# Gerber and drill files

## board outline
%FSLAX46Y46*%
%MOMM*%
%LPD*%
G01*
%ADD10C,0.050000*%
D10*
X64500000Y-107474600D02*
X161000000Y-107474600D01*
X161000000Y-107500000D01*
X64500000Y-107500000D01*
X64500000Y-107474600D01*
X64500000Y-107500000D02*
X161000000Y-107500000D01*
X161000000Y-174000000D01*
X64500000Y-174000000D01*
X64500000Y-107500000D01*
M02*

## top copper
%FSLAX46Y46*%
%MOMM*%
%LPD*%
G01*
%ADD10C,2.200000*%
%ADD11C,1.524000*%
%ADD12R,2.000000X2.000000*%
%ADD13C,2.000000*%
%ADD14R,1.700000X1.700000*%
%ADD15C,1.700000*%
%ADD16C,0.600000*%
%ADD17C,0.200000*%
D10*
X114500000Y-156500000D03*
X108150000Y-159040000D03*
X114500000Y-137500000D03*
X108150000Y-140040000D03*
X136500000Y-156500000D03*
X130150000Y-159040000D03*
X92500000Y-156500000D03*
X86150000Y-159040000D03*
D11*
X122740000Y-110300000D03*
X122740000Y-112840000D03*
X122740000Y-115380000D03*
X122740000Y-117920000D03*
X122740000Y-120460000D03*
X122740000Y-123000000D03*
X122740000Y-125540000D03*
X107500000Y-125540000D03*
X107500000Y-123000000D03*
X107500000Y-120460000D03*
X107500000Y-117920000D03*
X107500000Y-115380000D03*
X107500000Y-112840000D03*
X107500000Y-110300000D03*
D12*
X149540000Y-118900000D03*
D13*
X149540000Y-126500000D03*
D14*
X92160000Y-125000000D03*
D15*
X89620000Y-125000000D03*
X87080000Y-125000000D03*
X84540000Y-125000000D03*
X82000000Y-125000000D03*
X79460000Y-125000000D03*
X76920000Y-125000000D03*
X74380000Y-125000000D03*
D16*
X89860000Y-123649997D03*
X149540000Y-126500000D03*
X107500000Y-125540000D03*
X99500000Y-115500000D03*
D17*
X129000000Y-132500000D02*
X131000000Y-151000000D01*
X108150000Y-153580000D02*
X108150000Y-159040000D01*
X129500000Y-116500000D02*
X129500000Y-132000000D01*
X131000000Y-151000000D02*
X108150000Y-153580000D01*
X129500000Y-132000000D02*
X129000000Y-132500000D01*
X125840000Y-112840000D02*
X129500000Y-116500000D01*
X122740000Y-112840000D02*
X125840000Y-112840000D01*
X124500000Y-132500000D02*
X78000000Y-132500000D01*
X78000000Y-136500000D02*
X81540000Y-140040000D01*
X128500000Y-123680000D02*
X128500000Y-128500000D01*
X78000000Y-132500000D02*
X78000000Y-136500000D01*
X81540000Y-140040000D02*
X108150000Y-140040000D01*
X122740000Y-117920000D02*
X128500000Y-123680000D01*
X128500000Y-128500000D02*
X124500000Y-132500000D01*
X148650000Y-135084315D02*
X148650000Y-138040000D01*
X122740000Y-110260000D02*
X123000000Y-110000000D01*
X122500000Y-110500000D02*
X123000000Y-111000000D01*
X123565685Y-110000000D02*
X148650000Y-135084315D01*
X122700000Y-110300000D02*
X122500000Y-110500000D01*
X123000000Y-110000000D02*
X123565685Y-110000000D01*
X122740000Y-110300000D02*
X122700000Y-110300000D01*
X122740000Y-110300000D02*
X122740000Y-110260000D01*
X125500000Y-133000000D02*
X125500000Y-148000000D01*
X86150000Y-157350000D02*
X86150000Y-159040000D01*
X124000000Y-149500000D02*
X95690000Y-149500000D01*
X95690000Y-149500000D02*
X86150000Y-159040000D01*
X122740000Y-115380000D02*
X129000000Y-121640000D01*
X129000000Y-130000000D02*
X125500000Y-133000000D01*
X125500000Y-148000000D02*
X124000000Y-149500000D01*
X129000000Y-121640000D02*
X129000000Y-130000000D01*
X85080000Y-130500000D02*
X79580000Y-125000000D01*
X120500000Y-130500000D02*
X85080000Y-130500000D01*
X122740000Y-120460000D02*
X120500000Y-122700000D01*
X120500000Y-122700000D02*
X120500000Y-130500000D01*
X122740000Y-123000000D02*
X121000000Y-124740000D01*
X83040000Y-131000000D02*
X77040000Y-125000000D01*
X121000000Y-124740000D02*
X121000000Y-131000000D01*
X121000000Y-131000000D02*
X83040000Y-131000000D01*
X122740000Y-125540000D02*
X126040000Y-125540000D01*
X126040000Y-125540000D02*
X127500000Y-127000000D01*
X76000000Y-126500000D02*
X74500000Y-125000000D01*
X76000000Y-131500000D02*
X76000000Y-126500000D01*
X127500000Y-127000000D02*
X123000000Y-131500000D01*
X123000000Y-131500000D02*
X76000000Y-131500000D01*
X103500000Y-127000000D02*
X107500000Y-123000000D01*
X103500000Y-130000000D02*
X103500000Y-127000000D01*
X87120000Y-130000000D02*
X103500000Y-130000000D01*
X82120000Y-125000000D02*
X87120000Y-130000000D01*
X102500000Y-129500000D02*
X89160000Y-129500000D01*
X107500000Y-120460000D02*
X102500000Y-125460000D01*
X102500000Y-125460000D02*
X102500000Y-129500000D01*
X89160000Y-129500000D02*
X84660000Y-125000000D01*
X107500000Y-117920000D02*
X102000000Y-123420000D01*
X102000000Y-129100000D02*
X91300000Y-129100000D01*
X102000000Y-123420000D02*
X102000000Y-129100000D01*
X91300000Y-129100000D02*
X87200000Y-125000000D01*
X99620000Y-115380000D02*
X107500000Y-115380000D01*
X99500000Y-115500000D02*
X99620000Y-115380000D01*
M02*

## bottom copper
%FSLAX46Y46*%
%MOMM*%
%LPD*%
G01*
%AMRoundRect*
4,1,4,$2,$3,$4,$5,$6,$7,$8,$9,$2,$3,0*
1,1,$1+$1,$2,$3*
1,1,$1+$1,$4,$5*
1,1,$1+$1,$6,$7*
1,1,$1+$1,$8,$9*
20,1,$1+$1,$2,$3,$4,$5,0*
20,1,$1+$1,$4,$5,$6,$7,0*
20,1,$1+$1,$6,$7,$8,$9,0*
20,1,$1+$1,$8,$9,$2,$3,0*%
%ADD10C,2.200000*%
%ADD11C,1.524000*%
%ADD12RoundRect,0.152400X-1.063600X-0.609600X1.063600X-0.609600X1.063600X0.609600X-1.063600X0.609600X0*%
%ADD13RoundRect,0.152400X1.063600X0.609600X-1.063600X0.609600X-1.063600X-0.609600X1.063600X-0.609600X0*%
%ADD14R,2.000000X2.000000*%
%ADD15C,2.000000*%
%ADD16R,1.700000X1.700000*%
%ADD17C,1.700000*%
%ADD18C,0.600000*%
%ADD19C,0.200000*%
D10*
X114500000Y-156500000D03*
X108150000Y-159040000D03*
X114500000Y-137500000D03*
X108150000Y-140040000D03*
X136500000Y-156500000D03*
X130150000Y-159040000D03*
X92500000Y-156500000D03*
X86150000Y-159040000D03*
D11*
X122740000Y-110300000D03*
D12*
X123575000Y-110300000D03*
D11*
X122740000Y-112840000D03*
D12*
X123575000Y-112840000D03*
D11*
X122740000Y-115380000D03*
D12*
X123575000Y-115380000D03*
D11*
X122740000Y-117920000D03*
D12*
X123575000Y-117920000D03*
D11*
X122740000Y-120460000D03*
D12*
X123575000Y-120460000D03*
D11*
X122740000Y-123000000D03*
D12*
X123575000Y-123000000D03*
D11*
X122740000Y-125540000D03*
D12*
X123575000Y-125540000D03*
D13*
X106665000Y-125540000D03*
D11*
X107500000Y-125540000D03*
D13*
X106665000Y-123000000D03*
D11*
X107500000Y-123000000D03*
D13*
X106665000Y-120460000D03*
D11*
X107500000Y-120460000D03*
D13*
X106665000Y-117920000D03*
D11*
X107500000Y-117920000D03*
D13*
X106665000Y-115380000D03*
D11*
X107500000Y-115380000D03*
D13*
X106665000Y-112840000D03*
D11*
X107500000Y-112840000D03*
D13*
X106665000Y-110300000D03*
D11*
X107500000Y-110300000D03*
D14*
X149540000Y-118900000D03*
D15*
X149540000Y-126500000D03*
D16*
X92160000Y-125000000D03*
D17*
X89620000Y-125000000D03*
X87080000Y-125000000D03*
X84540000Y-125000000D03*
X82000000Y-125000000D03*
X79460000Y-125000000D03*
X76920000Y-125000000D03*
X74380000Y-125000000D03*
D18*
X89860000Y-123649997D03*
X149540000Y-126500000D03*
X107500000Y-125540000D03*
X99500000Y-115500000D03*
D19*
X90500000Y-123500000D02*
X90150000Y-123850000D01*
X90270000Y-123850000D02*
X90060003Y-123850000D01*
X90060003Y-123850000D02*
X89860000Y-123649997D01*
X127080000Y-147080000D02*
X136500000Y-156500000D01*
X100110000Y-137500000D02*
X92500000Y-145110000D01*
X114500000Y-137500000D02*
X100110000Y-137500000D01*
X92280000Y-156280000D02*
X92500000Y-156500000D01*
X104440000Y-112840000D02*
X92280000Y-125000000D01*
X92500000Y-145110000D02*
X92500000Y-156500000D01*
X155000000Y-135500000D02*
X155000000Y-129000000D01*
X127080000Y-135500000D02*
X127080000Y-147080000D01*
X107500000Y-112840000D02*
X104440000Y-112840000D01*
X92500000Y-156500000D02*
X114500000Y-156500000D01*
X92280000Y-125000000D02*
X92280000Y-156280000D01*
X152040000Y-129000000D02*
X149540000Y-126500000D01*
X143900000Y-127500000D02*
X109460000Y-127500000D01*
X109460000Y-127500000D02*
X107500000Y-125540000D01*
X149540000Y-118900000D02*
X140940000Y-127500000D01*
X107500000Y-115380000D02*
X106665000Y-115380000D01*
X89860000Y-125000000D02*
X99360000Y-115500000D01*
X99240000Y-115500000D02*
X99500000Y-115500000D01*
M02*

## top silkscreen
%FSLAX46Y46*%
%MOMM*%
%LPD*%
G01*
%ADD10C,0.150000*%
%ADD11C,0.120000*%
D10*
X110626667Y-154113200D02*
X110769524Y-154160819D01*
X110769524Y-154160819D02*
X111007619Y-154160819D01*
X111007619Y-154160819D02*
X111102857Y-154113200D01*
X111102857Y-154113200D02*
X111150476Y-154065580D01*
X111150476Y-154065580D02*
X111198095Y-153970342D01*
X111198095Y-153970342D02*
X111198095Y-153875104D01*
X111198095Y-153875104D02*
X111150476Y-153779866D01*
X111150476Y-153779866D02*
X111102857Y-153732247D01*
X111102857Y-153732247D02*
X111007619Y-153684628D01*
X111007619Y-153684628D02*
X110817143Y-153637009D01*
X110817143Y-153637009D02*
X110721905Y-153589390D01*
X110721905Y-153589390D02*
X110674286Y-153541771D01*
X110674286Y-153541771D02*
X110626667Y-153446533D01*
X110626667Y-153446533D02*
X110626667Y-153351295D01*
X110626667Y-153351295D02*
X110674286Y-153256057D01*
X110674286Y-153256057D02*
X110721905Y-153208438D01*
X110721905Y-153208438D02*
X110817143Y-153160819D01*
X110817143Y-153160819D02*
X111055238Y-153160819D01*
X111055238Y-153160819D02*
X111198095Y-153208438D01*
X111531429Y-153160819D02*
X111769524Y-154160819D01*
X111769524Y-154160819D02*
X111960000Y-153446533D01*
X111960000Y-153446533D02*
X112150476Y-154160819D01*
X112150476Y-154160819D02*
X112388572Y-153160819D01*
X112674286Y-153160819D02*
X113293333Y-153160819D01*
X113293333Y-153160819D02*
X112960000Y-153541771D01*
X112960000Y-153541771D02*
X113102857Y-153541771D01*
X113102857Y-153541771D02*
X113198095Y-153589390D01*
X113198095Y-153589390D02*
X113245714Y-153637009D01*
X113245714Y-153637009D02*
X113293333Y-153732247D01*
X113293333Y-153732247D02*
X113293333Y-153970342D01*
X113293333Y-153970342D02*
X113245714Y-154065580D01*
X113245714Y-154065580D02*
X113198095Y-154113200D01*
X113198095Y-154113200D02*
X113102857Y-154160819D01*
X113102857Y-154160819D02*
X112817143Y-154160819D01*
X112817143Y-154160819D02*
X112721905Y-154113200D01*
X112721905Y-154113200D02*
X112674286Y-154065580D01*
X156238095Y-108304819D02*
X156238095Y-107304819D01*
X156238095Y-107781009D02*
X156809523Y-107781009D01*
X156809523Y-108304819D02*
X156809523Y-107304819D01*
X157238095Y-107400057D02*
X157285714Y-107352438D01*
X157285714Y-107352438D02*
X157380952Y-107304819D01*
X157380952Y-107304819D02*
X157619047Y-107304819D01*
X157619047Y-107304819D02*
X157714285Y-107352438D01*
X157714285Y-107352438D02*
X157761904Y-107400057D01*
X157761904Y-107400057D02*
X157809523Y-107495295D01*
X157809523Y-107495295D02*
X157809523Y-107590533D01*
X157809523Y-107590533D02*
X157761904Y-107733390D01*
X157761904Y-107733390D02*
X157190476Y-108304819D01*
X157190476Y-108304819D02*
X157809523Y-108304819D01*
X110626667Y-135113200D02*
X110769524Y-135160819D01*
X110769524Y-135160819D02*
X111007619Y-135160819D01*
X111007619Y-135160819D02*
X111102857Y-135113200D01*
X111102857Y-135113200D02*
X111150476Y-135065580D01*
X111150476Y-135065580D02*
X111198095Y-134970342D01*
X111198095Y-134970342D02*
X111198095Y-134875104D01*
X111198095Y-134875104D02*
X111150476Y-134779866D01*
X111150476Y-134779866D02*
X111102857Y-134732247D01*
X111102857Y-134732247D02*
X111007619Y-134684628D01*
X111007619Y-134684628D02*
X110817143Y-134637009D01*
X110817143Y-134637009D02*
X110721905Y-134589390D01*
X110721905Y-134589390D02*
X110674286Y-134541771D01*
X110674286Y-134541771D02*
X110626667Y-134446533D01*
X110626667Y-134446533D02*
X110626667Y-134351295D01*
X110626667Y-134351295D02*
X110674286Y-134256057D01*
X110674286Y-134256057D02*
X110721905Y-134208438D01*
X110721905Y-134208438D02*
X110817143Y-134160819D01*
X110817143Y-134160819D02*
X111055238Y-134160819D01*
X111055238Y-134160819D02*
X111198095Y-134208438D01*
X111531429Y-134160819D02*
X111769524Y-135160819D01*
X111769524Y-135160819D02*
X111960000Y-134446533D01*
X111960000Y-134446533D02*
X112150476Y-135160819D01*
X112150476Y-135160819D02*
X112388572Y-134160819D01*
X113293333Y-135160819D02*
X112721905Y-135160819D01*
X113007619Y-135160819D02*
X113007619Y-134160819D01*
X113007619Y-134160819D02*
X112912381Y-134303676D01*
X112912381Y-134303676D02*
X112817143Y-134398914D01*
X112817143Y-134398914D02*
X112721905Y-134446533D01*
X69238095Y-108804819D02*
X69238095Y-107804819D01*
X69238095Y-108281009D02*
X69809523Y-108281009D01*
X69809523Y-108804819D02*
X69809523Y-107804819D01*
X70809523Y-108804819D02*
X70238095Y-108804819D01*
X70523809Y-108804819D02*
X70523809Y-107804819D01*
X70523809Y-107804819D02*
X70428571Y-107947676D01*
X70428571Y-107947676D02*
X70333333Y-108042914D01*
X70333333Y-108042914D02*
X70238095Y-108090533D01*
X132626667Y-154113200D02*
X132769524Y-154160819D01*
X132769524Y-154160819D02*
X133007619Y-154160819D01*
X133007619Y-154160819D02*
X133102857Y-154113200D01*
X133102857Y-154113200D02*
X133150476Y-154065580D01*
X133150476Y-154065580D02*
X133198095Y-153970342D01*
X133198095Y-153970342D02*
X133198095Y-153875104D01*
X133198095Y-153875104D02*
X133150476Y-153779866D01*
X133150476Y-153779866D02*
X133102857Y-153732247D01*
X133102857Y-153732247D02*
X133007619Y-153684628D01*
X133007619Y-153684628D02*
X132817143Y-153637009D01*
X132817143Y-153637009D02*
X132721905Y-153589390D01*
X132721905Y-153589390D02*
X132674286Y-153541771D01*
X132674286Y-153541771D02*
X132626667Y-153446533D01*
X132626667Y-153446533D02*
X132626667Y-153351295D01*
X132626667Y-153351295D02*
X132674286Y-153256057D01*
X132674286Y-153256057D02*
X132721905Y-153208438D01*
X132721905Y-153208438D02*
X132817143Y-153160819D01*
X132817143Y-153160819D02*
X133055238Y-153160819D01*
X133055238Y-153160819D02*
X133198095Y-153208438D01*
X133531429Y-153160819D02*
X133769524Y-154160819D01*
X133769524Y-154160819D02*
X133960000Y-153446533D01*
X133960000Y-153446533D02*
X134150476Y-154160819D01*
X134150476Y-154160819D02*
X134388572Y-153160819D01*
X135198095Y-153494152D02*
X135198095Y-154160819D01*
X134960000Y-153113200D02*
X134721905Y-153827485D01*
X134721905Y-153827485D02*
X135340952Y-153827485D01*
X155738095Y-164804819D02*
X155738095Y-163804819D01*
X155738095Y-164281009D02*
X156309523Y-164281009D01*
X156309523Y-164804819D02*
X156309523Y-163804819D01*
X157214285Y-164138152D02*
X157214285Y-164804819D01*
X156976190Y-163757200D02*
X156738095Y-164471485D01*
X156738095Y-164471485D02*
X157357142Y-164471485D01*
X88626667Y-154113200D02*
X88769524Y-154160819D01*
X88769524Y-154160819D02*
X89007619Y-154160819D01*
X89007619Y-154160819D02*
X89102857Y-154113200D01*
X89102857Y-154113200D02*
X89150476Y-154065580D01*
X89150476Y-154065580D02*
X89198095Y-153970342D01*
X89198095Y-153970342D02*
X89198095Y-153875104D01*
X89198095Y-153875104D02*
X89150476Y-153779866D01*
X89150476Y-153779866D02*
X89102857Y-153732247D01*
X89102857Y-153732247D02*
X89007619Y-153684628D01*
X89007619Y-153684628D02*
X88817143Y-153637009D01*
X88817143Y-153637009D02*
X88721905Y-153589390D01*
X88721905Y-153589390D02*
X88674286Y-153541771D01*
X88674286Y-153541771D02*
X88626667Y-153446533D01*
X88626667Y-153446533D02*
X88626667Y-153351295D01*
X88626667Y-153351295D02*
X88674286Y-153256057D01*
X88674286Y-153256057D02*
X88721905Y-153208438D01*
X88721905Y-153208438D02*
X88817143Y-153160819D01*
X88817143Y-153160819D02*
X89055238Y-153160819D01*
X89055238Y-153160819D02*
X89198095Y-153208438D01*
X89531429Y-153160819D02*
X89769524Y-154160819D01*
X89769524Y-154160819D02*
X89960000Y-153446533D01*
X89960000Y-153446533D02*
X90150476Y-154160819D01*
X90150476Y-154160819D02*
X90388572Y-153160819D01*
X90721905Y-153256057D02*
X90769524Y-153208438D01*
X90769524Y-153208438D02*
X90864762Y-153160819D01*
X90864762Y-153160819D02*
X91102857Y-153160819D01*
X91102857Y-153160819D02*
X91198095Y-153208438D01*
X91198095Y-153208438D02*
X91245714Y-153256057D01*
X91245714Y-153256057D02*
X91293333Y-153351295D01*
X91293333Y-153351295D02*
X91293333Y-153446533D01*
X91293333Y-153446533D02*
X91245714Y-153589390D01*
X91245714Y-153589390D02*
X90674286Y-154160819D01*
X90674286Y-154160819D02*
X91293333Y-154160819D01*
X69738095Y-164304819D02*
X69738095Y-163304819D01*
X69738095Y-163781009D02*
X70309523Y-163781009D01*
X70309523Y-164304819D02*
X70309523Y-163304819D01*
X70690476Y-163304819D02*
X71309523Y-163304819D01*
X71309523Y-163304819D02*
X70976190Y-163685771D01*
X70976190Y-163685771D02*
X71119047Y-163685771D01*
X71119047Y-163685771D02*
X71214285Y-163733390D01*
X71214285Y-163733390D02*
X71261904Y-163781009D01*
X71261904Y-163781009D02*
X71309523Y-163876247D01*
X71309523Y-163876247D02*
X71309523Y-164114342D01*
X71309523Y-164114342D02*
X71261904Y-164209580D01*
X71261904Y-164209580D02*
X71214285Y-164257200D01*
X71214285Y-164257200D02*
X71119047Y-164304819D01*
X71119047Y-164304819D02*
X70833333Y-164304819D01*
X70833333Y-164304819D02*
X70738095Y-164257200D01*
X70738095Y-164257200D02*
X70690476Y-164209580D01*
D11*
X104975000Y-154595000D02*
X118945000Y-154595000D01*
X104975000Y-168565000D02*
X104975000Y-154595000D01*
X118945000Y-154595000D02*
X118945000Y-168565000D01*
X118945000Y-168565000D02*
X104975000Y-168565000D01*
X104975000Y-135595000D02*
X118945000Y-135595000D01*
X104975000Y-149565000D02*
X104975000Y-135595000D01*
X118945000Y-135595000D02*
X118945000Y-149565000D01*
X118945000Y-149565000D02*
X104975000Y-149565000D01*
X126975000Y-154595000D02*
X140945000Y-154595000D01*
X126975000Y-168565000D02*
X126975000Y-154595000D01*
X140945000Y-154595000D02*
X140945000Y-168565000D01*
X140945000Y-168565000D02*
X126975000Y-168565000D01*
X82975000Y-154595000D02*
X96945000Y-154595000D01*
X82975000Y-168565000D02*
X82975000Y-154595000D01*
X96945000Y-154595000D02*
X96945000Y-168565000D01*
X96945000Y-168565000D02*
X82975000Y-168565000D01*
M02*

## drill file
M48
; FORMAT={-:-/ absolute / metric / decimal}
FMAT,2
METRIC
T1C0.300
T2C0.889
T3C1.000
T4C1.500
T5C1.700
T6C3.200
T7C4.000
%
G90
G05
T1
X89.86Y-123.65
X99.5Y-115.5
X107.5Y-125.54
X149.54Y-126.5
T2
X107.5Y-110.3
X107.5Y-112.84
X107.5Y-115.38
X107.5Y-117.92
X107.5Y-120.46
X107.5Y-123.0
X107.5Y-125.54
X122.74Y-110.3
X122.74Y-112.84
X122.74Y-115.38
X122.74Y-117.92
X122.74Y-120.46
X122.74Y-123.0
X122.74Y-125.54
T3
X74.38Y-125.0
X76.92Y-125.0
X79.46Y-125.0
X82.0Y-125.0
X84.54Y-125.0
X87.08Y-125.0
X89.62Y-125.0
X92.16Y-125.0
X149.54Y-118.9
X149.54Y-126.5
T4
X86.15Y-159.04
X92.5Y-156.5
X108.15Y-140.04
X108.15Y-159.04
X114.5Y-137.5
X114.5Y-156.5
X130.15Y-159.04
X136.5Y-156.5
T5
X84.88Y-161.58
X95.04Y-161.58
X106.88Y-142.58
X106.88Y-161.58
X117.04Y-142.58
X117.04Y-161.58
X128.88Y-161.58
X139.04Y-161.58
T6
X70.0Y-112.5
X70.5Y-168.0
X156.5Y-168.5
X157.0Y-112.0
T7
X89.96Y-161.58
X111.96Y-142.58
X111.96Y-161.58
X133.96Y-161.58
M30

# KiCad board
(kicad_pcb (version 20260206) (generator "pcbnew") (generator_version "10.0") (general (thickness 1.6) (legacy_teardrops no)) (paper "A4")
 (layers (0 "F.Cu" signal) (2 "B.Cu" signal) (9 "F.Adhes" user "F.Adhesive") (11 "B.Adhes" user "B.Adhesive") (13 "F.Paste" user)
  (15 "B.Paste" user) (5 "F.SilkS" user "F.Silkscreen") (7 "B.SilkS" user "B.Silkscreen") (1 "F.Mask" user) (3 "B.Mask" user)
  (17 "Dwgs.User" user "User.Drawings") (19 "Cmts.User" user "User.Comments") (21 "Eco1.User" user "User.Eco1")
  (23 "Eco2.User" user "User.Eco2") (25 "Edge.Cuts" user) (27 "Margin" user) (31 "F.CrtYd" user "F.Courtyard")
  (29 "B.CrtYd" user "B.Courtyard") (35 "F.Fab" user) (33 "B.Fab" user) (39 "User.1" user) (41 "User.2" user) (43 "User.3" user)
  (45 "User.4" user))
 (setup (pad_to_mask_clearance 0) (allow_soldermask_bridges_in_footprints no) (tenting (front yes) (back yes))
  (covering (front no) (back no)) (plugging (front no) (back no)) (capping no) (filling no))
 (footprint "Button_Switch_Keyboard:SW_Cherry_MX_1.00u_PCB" (layer "F.Cu") (at 114.5 156.5)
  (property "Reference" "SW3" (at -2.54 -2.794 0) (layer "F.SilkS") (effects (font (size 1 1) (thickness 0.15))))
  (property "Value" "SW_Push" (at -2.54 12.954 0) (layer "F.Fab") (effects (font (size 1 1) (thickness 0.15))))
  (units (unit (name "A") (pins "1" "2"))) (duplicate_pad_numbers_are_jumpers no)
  (fp_line (start -9.525 -1.905) (end 4.445 -1.905) (stroke (width 0.12) (type solid)) (layer "F.SilkS"))
  (fp_line (start -9.525 12.065) (end -9.525 -1.905) (stroke (width 0.12) (type solid)) (layer "F.SilkS"))
  (fp_line (start 4.445 -1.905) (end 4.445 12.065) (stroke (width 0.12) (type solid)) (layer "F.SilkS"))
  (fp_line (start 4.445 12.065) (end -9.525 12.065) (stroke (width 0.12) (type solid)) (layer "F.SilkS"))
  (pad "" np_thru_hole circle (at -7.62 5.08) (size 1.7 1.7) (drill 1.7) (layers "*.Cu" "*.Mask"))
  (pad "" np_thru_hole circle (at -2.54 5.08) (size 4 4) (drill 4) (layers "*.Cu" "*.Mask"))
  (pad "" np_thru_hole circle (at 2.54 5.08) (size 1.7 1.7) (drill 1.7) (layers "*.Cu" "*.Mask"))
  (pad "1" thru_hole circle (at 0 0) (size 2.2 2.2) (drill 1.5) (layers "*.Cu" "*.Mask") (remove_unused_layers no) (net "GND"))
  (pad "2" thru_hole circle (at -6.35 2.54) (size 2.2 2.2) (drill 1.5) (layers "*.Cu" "*.Mask") (remove_unused_layers no)
   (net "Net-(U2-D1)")))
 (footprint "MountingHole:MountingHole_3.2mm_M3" (layer "F.Cu") (at 157 112)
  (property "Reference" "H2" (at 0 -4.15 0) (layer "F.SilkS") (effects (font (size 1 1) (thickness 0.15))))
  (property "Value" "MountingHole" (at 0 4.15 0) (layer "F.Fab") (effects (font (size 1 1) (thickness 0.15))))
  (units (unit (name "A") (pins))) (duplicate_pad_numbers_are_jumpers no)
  (pad "" np_thru_hole circle (at 0 0) (size 3.2 3.2) (drill 3.2) (layers "*.Cu" "*.Mask")))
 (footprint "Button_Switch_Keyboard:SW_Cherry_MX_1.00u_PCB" (layer "F.Cu") (at 114.5 137.5)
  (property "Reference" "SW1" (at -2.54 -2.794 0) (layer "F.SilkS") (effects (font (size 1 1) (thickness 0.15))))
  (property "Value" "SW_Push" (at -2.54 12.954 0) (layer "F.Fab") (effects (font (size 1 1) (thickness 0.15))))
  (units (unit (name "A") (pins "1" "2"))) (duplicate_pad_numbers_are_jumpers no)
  (fp_line (start -9.525 -1.905) (end 4.445 -1.905) (stroke (width 0.12) (type solid)) (layer "F.SilkS"))
  (fp_line (start -9.525 12.065) (end -9.525 -1.905) (stroke (width 0.12) (type solid)) (layer "F.SilkS"))
  (fp_line (start 4.445 -1.905) (end 4.445 12.065) (stroke (width 0.12) (type solid)) (layer "F.SilkS"))
  (fp_line (start 4.445 12.065) (end -9.525 12.065) (stroke (width 0.12) (type solid)) (layer "F.SilkS"))
  (pad "" np_thru_hole circle (at -7.62 5.08) (size 1.7 1.7) (drill 1.7) (layers "*.Cu" "*.Mask"))
  (pad "" np_thru_hole circle (at -2.54 5.08) (size 4 4) (drill 4) (layers "*.Cu" "*.Mask"))
  (pad "" np_thru_hole circle (at 2.54 5.08) (size 1.7 1.7) (drill 1.7) (layers "*.Cu" "*.Mask"))
  (pad "1" thru_hole circle (at 0 0) (size 2.2 2.2) (drill 1.5) (layers "*.Cu" "*.Mask") (remove_unused_layers no) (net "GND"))
  (pad "2" thru_hole circle (at -6.35 2.54) (size 2.2 2.2) (drill 1.5) (layers "*.Cu" "*.Mask") (remove_unused_layers no)
   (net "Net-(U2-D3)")))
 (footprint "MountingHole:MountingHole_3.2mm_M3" (layer "F.Cu") (at 70 112.5)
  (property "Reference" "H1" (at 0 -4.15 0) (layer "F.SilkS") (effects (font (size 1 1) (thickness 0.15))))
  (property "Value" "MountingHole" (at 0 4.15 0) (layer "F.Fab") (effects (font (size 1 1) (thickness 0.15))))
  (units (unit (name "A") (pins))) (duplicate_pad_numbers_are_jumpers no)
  (pad "" np_thru_hole circle (at 0 0) (size 3.2 3.2) (drill 3.2) (layers "*.Cu" "*.Mask")))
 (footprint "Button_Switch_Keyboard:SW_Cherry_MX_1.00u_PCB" (layer "F.Cu") (at 136.5 156.5)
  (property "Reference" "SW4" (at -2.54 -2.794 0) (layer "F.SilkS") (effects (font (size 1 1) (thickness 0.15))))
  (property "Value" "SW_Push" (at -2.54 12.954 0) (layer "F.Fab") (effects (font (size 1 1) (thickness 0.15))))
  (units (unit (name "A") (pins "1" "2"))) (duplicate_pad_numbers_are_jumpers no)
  (fp_line (start -9.525 -1.905) (end 4.445 -1.905) (stroke (width 0.12) (type solid)) (layer "F.SilkS"))
  (fp_line (start -9.525 12.065) (end -9.525 -1.905) (stroke (width 0.12) (type solid)) (layer "F.SilkS"))
  (fp_line (start 4.445 -1.905) (end 4.445 12.065) (stroke (width 0.12) (type solid)) (layer "F.SilkS"))
  (fp_line (start 4.445 12.065) (end -9.525 12.065) (stroke (width 0.12) (type solid)) (layer "F.SilkS"))
  (pad "" np_thru_hole circle (at -7.62 5.08) (size 1.7 1.7) (drill 1.7) (layers "*.Cu" "*.Mask"))
  (pad "" np_thru_hole circle (at -2.54 5.08) (size 4 4) (drill 4) (layers "*.Cu" "*.Mask"))
  (pad "" np_thru_hole circle (at 2.54 5.08) (size 1.7 1.7) (drill 1.7) (layers "*.Cu" "*.Mask"))
  (pad "1" thru_hole circle (at 0 0) (size 2.2 2.2) (drill 1.5) (layers "*.Cu" "*.Mask") (remove_unused_layers no) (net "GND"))
  (pad "2" thru_hole circle (at -6.35 2.54) (size 2.2 2.2) (drill 1.5) (layers "*.Cu" "*.Mask") (remove_unused_layers no)
   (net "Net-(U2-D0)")))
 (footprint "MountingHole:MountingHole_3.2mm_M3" (layer "F.Cu") (at 156.5 168.5)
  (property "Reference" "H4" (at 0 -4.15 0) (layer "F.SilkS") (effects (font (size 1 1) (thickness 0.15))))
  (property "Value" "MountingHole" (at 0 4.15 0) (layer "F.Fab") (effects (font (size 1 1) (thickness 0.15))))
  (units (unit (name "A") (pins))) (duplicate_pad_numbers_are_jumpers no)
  (pad "" np_thru_hole circle (at 0 0) (size 3.2 3.2) (drill 3.2) (layers "*.Cu" "*.Mask")))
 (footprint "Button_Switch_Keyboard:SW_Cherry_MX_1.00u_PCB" (layer "F.Cu") (at 92.5 156.5)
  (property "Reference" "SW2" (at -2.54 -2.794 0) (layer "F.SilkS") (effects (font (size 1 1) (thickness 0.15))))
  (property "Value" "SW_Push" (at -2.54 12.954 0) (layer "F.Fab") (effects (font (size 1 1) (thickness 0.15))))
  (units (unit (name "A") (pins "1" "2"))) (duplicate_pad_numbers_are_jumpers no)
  (fp_line (start -9.525 -1.905) (end 4.445 -1.905) (stroke (width 0.12) (type solid)) (layer "F.SilkS"))
  (fp_line (start -9.525 12.065) (end -9.525 -1.905) (stroke (width 0.12) (type solid)) (layer "F.SilkS"))
  (fp_line (start 4.445 -1.905) (end 4.445 12.065) (stroke (width 0.12) (type solid)) (layer "F.SilkS"))
  (fp_line (start 4.445 12.065) (end -9.525 12.065) (stroke (width 0.12) (type solid)) (layer "F.SilkS"))
  (pad "" np_thru_hole circle (at -7.62 5.08) (size 1.7 1.7) (drill 1.7) (layers "*.Cu" "*.Mask"))
  (pad "" np_thru_hole circle (at -2.54 5.08) (size 4 4) (drill 4) (layers "*.Cu" "*.Mask"))
  (pad "" np_thru_hole circle (at 2.54 5.08) (size 1.7 1.7) (drill 1.7) (layers "*.Cu" "*.Mask"))
  (pad "1" thru_hole circle (at 0 0) (size 2.2 2.2) (drill 1.5) (layers "*.Cu" "*.Mask") (remove_unused_layers no) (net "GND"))
  (pad "2" thru_hole circle (at -6.35 2.54) (size 2.2 2.2) (drill 1.5) (layers "*.Cu" "*.Mask") (remove_unused_layers no)
   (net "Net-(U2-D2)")))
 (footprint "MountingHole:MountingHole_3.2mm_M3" (layer "F.Cu") (at 70.5 168)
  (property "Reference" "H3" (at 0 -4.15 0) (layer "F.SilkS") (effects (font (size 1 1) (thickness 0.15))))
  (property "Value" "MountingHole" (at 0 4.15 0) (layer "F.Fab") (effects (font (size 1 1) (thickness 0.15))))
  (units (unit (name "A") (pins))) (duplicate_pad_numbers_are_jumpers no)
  (pad "" np_thru_hole circle (at 0 0) (size 3.2 3.2) (drill 3.2) (layers "*.Cu" "*.Mask")))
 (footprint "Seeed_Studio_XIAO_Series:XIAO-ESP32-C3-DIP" (layer "B.Cu") (at 115.12 117.92 90)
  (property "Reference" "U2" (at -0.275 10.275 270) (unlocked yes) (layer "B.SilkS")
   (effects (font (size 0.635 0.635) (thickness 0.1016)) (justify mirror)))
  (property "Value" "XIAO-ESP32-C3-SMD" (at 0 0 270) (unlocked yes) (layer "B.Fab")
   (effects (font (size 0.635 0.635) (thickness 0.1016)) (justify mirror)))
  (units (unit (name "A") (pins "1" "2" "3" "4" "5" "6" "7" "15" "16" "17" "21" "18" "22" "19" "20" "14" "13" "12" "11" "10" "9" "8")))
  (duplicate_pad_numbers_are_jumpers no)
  (pad "1" thru_hole circle (at 7.62 7.62) (size 1.524 1.524) (drill 0.889) (layers "*.Cu" "*.Mask") (remove_unused_layers no)
   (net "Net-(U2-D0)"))
  (pad "1" smd roundrect (at 7.62 8.455) (size 2.432 1.524) (layers "B.Cu" "B.Mask") (roundrect_rratio 0.1) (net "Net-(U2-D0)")
   (thermal_bridge_angle 45))
  (pad "2" thru_hole circle (at 5.08 7.62) (size 1.524 1.524) (drill 0.889) (layers "*.Cu" "*.Mask") (remove_unused_layers no)
   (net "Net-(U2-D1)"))
  (pad "2" smd roundrect (at 5.08 8.455) (size 2.432 1.524) (layers "B.Cu" "B.Mask") (roundrect_rratio 0.1) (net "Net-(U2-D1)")
   (thermal_bridge_angle 45))
  (pad "3" thru_hole circle (at 2.54 7.62) (size 1.524 1.524) (drill 0.889) (layers "*.Cu" "*.Mask") (remove_unused_layers no)
   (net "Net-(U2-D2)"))
  (pad "3" smd roundrect (at 2.54 8.455) (size 2.432 1.524) (layers "B.Cu" "B.Mask") (roundrect_rratio 0.1) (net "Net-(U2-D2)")
   (thermal_bridge_angle 45))
  (pad "4" thru_hole circle (at 0 7.62) (size 1.524 1.524) (drill 0.889) (layers "*.Cu" "*.Mask") (remove_unused_layers no)
   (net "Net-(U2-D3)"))
  (pad "4" smd roundrect (at 0 8.455) (size 2.432 1.524) (layers "B.Cu" "B.Mask") (roundrect_rratio 0.1) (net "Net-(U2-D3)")
   (thermal_bridge_angle 45))
  (pad "5" thru_hole circle (at -2.54 7.62) (size 1.524 1.524) (drill 0.889) (layers "*.Cu" "*.Mask") (remove_unused_layers no) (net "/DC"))
  (pad "5" smd roundrect (at -2.54 8.455) (size 2.432 1.524) (layers "B.Cu" "B.Mask") (roundrect_rratio 0.1) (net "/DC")
   (thermal_bridge_angle 45))
  (pad "6" thru_hole circle (at -5.08 7.62) (size 1.524 1.524) (drill 0.889) (layers "*.Cu" "*.Mask") (remove_unused_layers no) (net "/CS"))
  (pad "6" smd roundrect (at -5.08 8.455) (size 2.432 1.524) (layers "B.Cu" "B.Mask") (roundrect_rratio 0.1) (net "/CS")
   (thermal_bridge_angle 45))
  (pad "7" thru_hole circle (at -7.62 7.62) (size 1.524 1.524) (drill 0.889) (layers "*.Cu" "*.Mask") (remove_unused_layers no) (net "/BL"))
  (pad "7" smd roundrect (at -7.62 8.455) (size 2.432 1.524) (layers "B.Cu" "B.Mask") (roundrect_rratio 0.1) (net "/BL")
   (thermal_bridge_angle 45))
  (pad "8" smd roundrect (at -7.62 -8.455 180) (size 2.432 1.524) (layers "B.Cu" "B.Mask") (roundrect_rratio 0.1) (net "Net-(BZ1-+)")
   (thermal_bridge_angle 45))
  (pad "8" thru_hole circle (at -7.62 -7.62 180) (size 1.524 1.524) (drill 0.889) (layers "*.Cu" "*.Mask") (remove_unused_layers no)
   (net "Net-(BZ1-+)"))
  (pad "9" smd roundrect (at -5.08 -8.455 180) (size 2.432 1.524) (layers "B.Cu" "B.Mask") (roundrect_rratio 0.1) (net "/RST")
   (thermal_bridge_angle 45))
  (pad "9" thru_hole circle (at -5.08 -7.62 180) (size 1.524 1.524) (drill 0.889) (layers "*.Cu" "*.Mask") (remove_unused_layers no)
   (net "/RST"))
  (pad "10" smd roundrect (at -2.54 -8.455 180) (size 2.432 1.524) (layers "B.Cu" "B.Mask") (roundrect_rratio 0.1) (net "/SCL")
   (thermal_bridge_angle 45))
  (pad "10" thru_hole circle (at -2.54 -7.62 180) (size 1.524 1.524) (drill 0.889) (layers "*.Cu" "*.Mask") (remove_unused_layers no)
   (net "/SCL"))
  (pad "11" smd roundrect (at 0 -8.455 180) (size 2.432 1.524) (layers "B.Cu" "B.Mask") (roundrect_rratio 0.1) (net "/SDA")
   (thermal_bridge_angle 45))
  (pad "11" thru_hole circle (at 0 -7.62 180) (size 1.524 1.524) (drill 0.889) (layers "*.Cu" "*.Mask") (remove_unused_layers no)
   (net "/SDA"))
  (pad "12" smd roundrect (at 2.54 -8.455 180) (size 2.432 1.524) (layers "B.Cu" "B.Mask") (roundrect_rratio 0.1) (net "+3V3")
   (thermal_bridge_angle 45))
  (pad "12" thru_hole circle (at 2.54 -7.62 180) (size 1.524 1.524) (drill 0.889) (layers "*.Cu" "*.Mask") (remove_unused_layers no)
   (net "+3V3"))
  (pad "13" smd roundrect (at 5.08 -8.455 180) (size 2.432 1.524) (layers "B.Cu" "B.Mask") (roundrect_rratio 0.1) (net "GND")
   (thermal_bridge_angle 45))
  (pad "13" thru_hole circle (at 5.08 -7.62 180) (size 1.524 1.524) (drill 0.889) (layers "*.Cu" "*.Mask") (remove_unused_layers no)
   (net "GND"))
  (pad "14" smd roundrect (at 7.62 -8.455 180) (size 2.432 1.524) (layers "B.Cu" "B.Mask") (roundrect_rratio 0.1)
   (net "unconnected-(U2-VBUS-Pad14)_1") (thermal_bridge_angle 45))
  (pad "14" thru_hole circle (at 7.62 -7.62 180) (size 1.524 1.524) (drill 0.889) (layers "*.Cu" "*.Mask") (remove_unused_layers no)
   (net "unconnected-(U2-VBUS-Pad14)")))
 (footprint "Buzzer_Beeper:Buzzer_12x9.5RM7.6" (layer "B.Cu") (at 149.54 118.9 -90)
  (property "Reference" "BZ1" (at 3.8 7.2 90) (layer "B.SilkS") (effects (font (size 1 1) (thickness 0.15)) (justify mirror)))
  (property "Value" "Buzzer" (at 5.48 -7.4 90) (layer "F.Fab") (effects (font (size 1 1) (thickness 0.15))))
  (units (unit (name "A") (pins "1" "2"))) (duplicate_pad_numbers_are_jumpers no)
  (pad "1" thru_hole rect (at 0 0 270) (size 2 2) (drill 1) (layers "*.Cu" "*.Mask") (remove_unused_layers no) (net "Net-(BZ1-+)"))
  (pad "2" thru_hole circle (at 7.6 0 270) (size 2 2) (drill 1) (layers "*.Cu" "*.Mask") (remove_unused_layers no) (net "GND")))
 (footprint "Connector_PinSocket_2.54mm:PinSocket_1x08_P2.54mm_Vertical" (layer "B.Cu") (at 92.16 125 90)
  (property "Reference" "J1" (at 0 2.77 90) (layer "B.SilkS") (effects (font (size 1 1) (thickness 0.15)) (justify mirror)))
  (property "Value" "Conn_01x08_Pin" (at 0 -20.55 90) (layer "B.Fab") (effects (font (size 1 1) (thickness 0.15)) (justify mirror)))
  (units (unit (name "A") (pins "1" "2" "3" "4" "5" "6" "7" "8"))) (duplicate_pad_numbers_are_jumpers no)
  (pad "1" thru_hole rect (at 0 0 90) (size 1.7 1.7) (drill 1) (layers "*.Cu" "*.Mask") (remove_unused_layers no) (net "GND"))
  (pad "2" thru_hole circle (at 0 -2.54 90) (size 1.7 1.7) (drill 1) (layers "*.Cu" "*.Mask") (remove_unused_layers no) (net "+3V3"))
  (pad "3" thru_hole circle (at 0 -5.08 90) (size 1.7 1.7) (drill 1) (layers "*.Cu" "*.Mask") (remove_unused_layers no) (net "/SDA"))
  (pad "4" thru_hole circle (at 0 -7.62 90) (size 1.7 1.7) (drill 1) (layers "*.Cu" "*.Mask") (remove_unused_layers no) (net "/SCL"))
  (pad "5" thru_hole circle (at 0 -10.16 90) (size 1.7 1.7) (drill 1) (layers "*.Cu" "*.Mask") (remove_unused_layers no) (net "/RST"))
  (pad "6" thru_hole circle (at 0 -12.7 90) (size 1.7 1.7) (drill 1) (layers "*.Cu" "*.Mask") (remove_unused_layers no) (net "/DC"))
  (pad "7" thru_hole circle (at 0 -15.24 90) (size 1.7 1.7) (drill 1) (layers "*.Cu" "*.Mask") (remove_unused_layers no) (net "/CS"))
  (pad "8" thru_hole circle (at 0 -17.78 90) (size 1.7 1.7) (drill 1) (layers "*.Cu" "*.Mask") (remove_unused_layers no) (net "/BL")))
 (gr_rect (start 64.5 107.4746) (end 161 107.5) (stroke (width 0.05) (type default)) (fill no) (layer "Edge.Cuts"))
 (gr_rect (start 64.5 107.5) (end 161 174) (stroke (width 0.05) (type default)) (fill no) (layer "Edge.Cuts"))
 (via (at 89.86 123.649997) (size 0.6) (drill 0.3) (layers "F.Cu" "B.Cu") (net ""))
 (segment (start 90.5 123.5) (end 90.15 123.85) (width 0.2) (layer "B.Cu") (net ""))
 (segment (start 90.27 123.85) (end 90.060003 123.85) (width 0.2) (layer "B.Cu") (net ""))
 (segment (start 90.060003 123.85) (end 89.86 123.649997) (width 0.2) (layer "B.Cu") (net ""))
 (via (at 149.54 126.5) (size 0.6) (drill 0.3) (layers "F.Cu" "B.Cu") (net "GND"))
 (segment (start 127.08 147.08) (end 136.5 156.5) (width 0.2) (layer "B.Cu") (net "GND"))
 (segment (start 100.11 137.5) (end 92.5 145.11) (width 0.2) (layer "B.Cu") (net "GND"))
 (segment (start 114.5 137.5) (end 100.11 137.5) (width 0.2) (layer "B.Cu") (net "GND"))
 (segment (start 92.28 156.28) (end 92.5 156.5) (width 0.2) (layer "B.Cu") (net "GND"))
 (segment (start 104.44 112.84) (end 92.28 125) (width 0.2) (layer "B.Cu") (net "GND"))
 (segment (start 92.5 145.11) (end 92.5 156.5) (width 0.2) (layer "B.Cu") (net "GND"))
 (segment (start 155 135.5) (end 155 129) (width 0.2) (layer "B.Cu") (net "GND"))
 (segment (start 127.08 135.5) (end 127.08 147.08) (width 0.2) (layer "B.Cu") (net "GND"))
 (segment (start 107.5 112.84) (end 104.44 112.84) (width 0.2) (layer "B.Cu") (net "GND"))
 (segment (start 92.5 156.5) (end 114.5 156.5) (width 0.2) (layer "B.Cu") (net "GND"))
 (segment (start 92.28 125) (end 92.28 156.28) (width 0.2) (layer "B.Cu") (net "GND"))
 (segment (start 152.04 129) (end 149.54 126.5) (width 0.2) (layer "B.Cu") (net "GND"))
 (segment (start 129 132.5) (end 131 151) (width 0.2) (layer "F.Cu") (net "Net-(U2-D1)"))
 (segment (start 108.15 153.58) (end 108.15 159.04) (width 0.2) (layer "F.Cu") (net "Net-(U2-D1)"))
 (segment (start 129.5 116.5) (end 129.5 132) (width 0.2) (layer "F.Cu") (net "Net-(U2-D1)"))
 (segment (start 131 151) (end 108.15 153.58) (width 0.2) (layer "F.Cu") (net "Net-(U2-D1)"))
 (segment (start 129.5 132) (end 129 132.5) (width 0.2) (layer "F.Cu") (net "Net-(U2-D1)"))
 (segment (start 125.84 112.84) (end 129.5 116.5) (width 0.2) (layer "F.Cu") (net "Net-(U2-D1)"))
 (segment (start 122.74 112.84) (end 125.84 112.84) (width 0.2) (layer "F.Cu") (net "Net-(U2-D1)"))
 (segment (start 124.5 132.5) (end 78 132.5) (width 0.2) (layer "F.Cu") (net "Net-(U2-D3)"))
 (segment (start 78 136.5) (end 81.54 140.04) (width 0.2) (layer "F.Cu") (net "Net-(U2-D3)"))
 (segment (start 128.5 123.68) (end 128.5 128.5) (width 0.2) (layer "F.Cu") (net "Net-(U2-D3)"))
 (segment (start 78 132.5) (end 78 136.5) (width 0.2) (layer "F.Cu") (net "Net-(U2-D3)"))
 (segment (start 81.54 140.04) (end 108.15 140.04) (width 0.2) (layer "F.Cu") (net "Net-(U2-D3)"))
 (segment (start 122.74 117.92) (end 128.5 123.68) (width 0.2) (layer "F.Cu") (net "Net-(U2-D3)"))
 (segment (start 128.5 128.5) (end 124.5 132.5) (width 0.2) (layer "F.Cu") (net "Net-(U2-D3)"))
 (segment (start 148.65 135.084315) (end 148.65 138.04) (width 0.2) (layer "F.Cu") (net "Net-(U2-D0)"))
 (segment (start 122.74 110.26) (end 123 110) (width 0.2) (layer "F.Cu") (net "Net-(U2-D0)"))
 (segment (start 122.5 110.5) (end 123 111) (width 0.2) (layer "F.Cu") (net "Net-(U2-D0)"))
 (segment (start 123.565685 110) (end 148.65 135.084315) (width 0.2) (layer "F.Cu") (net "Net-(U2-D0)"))
 (segment (start 122.7 110.3) (end 122.5 110.5) (width 0.2) (layer "F.Cu") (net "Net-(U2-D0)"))
 (segment (start 123 110) (end 123.565685 110) (width 0.2) (layer "F.Cu") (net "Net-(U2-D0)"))
 (segment (start 122.74 110.3) (end 122.7 110.3) (width 0.2) (layer "F.Cu") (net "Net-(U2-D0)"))
 (segment (start 122.74 110.3) (end 122.74 110.26) (width 0.2) (layer "F.Cu") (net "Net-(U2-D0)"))
 (segment (start 125.5 133) (end 125.5 148) (width 0.2) (layer "F.Cu") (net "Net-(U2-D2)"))
 (segment (start 86.15 157.35) (end 86.15 159.04) (width 0.2) (layer "F.Cu") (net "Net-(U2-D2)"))
 (segment (start 124 149.5) (end 95.69 149.5) (width 0.2) (layer "F.Cu") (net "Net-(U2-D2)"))
 (segment (start 95.69 149.5) (end 86.15 159.04) (width 0.2) (layer "F.Cu") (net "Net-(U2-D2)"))
 (segment (start 122.74 115.38) (end 129 121.64) (width 0.2) (layer "F.Cu") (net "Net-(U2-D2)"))
 (segment (start 129 130) (end 125.5 133) (width 0.2) (layer "F.Cu") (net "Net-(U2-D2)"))
 (segment (start 125.5 148) (end 124 149.5) (width 0.2) (layer "F.Cu") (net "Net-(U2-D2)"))
 (segment (start 129 121.64) (end 129 130) (width 0.2) (layer "F.Cu") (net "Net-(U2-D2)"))
 (segment (start 85.08 130.5) (end 79.58 125) (width 0.2) (layer "F.Cu") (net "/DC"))
 (segment (start 120.5 130.5) (end 85.08 130.5) (width 0.2) (layer "F.Cu") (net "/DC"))
 (segment (start 122.74 120.46) (end 120.5 122.7) (width 0.2) (layer "F.Cu") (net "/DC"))
 (segment (start 120.5 122.7) (end 120.5 130.5) (width 0.2) (layer "F.Cu") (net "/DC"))
 (segment (start 122.74 123) (end 121 124.74) (width 0.2) (layer "F.Cu") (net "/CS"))
 (segment (start 83.04 131) (end 77.04 125) (width 0.2) (layer "F.Cu") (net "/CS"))
 (segment (start 121 124.74) (end 121 131) (width 0.2) (layer "F.Cu") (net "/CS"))
 (segment (start 121 131) (end 83.04 131) (width 0.2) (layer "F.Cu") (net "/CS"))
 (segment (start 122.74 125.54) (end 126.04 125.54) (width 0.2) (layer "F.Cu") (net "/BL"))
 (segment (start 126.04 125.54) (end 127.5 127) (width 0.2) (layer "F.Cu") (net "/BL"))
 (segment (start 76 126.5) (end 74.5 125) (width 0.2) (layer "F.Cu") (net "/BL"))
 (segment (start 76 131.5) (end 76 126.5) (width 0.2) (layer "F.Cu") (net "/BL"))
 (segment (start 127.5 127) (end 123 131.5) (width 0.2) (layer "F.Cu") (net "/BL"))
 (segment (start 123 131.5) (end 76 131.5) (width 0.2) (layer "F.Cu") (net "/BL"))
 (via (at 107.5 125.54) (size 0.6) (drill 0.3) (layers "F.Cu" "B.Cu") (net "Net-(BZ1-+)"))
 (segment (start 143.9 127.5) (end 109.46 127.5) (width 0.2) (layer "B.Cu") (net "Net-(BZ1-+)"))
 (segment (start 109.46 127.5) (end 107.5 125.54) (width 0.2) (layer "B.Cu") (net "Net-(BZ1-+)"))
 (segment (start 149.54 118.9) (end 140.94 127.5) (width 0.2) (layer "B.Cu") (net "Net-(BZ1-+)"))
 (segment (start 103.5 127) (end 107.5 123) (width 0.2) (layer "F.Cu") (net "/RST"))
 (segment (start 103.5 130) (end 103.5 127) (width 0.2) (layer "F.Cu") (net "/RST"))
 (segment (start 87.12 130) (end 103.5 130) (width 0.2) (layer "F.Cu") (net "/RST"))
 (segment (start 82.12 125) (end 87.12 130) (width 0.2) (layer "F.Cu") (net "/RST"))
 (segment (start 102.5 129.5) (end 89.16 129.5) (width 0.2) (layer "F.Cu") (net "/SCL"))
 (segment (start 107.5 120.46) (end 102.5 125.46) (width 0.2) (layer "F.Cu") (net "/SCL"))
 (segment (start 102.5 125.46) (end 102.5 129.5) (width 0.2) (layer "F.Cu") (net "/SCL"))
 (segment (start 89.16 129.5) (end 84.66 125) (width 0.2) (layer "F.Cu") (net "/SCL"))
 (segment (start 107.5 117.92) (end 102 123.42) (width 0.2) (layer "F.Cu") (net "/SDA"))
 (segment (start 102 129.1) (end 91.3 129.1) (width 0.2) (layer "F.Cu") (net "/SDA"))
 (segment (start 102 123.42) (end 102 129.1) (width 0.2) (layer "F.Cu") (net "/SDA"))
 (segment (start 91.3 129.1) (end 87.2 125) (width 0.2) (layer "F.Cu") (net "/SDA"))
 (segment (start 99.62 115.38) (end 107.5 115.38) (width 0.2) (layer "F.Cu") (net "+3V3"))
 (segment (start 99.5 115.5) (end 99.62 115.38) (width 0.2) (layer "F.Cu") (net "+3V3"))
 (via (at 99.5 115.5) (size 0.6) (drill 0.3) (layers "F.Cu" "B.Cu") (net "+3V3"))
 (segment (start 107.5 115.38) (end 106.665 115.38) (width 0.2) (layer "B.Cu") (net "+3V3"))
 (segment (start 89.86 125) (end 99.36 115.5) (width 0.2) (layer "B.Cu") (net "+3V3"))
 (segment (start 99.24 115.5) (end 99.5 115.5) (width 0.2) (layer "B.Cu") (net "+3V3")))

